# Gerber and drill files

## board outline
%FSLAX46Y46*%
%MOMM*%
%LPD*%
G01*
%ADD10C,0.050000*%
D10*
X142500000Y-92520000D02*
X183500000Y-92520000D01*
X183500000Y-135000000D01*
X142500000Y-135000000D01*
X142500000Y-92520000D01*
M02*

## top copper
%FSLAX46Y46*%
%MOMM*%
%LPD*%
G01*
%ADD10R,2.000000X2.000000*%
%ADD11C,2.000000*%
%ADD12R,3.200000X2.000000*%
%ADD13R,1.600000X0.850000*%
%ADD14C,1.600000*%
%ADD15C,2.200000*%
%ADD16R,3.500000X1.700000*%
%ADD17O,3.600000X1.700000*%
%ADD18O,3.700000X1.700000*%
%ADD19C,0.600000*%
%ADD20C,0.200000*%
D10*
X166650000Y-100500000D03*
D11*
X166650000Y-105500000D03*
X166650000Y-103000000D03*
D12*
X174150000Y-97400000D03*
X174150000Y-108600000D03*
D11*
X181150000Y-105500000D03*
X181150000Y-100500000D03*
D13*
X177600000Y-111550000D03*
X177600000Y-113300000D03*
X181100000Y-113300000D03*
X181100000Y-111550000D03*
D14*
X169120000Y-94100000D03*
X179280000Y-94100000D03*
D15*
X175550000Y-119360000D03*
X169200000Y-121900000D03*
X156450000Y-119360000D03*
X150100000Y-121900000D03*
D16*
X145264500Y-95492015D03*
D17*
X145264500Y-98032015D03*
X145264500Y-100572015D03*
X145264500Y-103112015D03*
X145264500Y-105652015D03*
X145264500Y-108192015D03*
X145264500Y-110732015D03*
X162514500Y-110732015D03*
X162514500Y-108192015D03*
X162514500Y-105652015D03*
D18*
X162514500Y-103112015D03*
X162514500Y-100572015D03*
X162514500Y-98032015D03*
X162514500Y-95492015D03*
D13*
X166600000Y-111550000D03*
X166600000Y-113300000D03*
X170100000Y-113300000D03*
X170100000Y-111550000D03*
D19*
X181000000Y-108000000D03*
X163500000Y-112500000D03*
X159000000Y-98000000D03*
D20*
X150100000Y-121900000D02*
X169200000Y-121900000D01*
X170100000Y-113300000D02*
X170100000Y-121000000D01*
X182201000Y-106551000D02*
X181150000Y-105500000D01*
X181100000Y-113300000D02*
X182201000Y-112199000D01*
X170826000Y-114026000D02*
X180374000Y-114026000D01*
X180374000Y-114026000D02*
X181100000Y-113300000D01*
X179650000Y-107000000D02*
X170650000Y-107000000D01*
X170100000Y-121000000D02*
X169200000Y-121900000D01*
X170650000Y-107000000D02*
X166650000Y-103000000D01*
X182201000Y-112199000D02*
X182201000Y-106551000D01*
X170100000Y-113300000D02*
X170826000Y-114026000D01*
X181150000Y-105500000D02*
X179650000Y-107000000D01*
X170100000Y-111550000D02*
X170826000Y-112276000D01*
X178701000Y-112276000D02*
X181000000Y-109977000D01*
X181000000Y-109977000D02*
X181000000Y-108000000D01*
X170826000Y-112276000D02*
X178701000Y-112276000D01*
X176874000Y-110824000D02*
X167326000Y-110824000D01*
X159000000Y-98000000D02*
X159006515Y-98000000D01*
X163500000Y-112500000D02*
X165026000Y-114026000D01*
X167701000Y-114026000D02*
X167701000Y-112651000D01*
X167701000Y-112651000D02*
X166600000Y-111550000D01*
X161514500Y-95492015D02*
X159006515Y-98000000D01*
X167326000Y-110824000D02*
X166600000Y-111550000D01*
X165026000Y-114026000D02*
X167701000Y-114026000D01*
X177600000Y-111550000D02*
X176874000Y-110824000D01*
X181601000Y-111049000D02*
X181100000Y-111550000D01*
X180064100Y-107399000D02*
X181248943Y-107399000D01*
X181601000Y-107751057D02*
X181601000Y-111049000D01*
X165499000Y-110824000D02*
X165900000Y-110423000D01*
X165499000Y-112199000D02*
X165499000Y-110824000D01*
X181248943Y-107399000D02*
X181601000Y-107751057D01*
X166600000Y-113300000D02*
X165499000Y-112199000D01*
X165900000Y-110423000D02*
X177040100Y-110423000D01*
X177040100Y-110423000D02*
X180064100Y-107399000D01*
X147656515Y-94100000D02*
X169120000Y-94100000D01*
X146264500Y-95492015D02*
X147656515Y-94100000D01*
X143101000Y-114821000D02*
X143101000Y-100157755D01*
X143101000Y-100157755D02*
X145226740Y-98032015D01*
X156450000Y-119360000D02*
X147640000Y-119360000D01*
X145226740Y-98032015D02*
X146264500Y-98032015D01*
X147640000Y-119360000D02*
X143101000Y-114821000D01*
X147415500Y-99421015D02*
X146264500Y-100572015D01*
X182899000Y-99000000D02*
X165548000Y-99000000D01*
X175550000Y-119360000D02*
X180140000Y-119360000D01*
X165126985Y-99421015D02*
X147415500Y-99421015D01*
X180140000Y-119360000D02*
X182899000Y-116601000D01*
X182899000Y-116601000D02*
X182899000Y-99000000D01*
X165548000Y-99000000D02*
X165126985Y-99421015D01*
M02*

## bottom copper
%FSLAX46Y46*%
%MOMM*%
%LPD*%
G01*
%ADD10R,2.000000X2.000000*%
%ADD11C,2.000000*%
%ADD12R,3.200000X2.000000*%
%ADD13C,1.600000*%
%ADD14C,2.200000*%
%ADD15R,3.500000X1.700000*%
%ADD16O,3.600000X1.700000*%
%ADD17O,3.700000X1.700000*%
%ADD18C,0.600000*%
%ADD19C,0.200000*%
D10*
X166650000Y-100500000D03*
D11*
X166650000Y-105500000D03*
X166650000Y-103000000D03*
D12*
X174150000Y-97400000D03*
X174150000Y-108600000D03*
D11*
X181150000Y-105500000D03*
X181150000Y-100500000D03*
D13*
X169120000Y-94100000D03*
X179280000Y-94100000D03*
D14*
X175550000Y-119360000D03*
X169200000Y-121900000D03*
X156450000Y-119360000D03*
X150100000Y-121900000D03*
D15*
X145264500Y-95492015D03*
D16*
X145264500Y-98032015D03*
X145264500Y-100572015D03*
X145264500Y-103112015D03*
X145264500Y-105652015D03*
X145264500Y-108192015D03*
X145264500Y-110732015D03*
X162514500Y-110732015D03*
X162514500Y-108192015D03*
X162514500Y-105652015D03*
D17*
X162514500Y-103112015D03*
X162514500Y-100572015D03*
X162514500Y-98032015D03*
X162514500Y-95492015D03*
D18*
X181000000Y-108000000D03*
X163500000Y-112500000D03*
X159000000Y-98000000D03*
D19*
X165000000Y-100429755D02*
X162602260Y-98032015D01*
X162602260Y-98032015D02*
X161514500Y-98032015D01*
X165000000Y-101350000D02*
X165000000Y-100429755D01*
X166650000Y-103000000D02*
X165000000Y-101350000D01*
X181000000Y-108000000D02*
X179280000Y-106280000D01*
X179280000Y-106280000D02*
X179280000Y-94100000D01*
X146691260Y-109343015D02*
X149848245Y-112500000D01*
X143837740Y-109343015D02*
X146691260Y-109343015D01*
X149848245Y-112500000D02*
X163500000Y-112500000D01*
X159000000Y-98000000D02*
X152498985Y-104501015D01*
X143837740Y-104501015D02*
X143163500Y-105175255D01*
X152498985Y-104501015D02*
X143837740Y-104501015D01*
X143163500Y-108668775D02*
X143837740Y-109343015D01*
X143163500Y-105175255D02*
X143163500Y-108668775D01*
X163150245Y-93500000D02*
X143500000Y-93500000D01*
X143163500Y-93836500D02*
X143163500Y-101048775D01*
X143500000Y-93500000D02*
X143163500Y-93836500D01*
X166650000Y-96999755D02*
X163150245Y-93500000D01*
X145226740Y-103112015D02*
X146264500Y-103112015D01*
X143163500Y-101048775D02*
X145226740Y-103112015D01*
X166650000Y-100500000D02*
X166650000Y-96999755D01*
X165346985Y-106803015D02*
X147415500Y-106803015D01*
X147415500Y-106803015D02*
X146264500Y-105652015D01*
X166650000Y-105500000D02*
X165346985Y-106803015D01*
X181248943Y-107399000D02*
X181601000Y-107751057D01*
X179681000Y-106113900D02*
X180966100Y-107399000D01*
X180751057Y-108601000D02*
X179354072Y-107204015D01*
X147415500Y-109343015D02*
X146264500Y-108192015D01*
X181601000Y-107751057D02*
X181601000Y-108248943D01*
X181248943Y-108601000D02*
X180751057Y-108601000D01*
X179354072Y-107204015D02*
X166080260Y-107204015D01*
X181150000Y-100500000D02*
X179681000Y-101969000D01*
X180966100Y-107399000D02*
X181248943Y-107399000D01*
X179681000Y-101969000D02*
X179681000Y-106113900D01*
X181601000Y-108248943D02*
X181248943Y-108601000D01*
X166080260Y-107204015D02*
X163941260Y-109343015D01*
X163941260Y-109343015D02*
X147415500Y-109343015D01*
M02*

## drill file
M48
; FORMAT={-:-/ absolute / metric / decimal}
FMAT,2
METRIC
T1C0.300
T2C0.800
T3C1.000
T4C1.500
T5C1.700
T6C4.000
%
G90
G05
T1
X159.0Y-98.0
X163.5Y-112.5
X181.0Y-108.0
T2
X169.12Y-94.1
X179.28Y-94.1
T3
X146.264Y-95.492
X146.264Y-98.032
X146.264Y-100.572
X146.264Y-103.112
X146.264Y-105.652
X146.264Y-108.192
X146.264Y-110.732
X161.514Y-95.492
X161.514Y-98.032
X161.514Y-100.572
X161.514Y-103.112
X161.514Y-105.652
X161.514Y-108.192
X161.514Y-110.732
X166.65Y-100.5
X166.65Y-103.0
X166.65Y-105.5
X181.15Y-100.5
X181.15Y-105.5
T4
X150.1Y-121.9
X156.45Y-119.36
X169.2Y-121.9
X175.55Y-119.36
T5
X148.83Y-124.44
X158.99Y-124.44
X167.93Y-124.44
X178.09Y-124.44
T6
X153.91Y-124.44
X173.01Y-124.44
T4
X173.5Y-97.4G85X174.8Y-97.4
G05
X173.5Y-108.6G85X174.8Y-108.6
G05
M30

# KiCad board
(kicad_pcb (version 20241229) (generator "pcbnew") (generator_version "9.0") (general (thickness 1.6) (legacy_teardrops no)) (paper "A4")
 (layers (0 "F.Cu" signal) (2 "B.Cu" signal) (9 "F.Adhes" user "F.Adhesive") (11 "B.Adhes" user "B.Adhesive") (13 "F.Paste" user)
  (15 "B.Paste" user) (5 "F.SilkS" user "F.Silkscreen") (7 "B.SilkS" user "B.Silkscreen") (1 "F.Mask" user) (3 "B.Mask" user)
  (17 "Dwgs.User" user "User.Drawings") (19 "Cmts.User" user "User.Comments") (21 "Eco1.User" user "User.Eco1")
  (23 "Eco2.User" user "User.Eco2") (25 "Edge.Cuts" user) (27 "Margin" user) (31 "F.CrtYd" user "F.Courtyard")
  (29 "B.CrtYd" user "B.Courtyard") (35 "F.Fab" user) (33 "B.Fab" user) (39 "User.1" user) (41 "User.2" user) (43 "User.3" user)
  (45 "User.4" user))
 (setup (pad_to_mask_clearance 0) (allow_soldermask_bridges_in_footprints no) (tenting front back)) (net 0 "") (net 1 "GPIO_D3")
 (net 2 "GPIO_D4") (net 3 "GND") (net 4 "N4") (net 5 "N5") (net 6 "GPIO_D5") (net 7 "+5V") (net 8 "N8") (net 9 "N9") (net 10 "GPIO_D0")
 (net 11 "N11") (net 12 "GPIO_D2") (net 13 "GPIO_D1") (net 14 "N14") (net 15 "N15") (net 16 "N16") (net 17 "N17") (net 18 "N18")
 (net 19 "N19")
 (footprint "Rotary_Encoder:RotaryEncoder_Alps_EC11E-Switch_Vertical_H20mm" (layer "F.Cu") (at 166.65 100.5)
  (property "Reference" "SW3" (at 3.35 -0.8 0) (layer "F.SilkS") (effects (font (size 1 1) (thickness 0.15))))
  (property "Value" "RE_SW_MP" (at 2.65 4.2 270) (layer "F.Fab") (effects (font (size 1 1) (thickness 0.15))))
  (pad "A" thru_hole rect (at 0 0) (size 2 2) (drill 1) (layers "*.Cu" "*.Mask") (remove_unused_layers no) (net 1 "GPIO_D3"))
  (pad "B" thru_hole circle (at 0 5) (size 2 2) (drill 1) (layers "*.Cu" "*.Mask") (remove_unused_layers no) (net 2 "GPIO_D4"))
  (pad "C" thru_hole circle (at 0 2.5) (size 2 2) (drill 1) (layers "*.Cu" "*.Mask") (remove_unused_layers no) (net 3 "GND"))
  (pad "MP" thru_hole rect (at 7.5 -3.1) (size 3.2 2) (drill oval 2.8 1.5) (layers "*.Cu" "*.Mask") (remove_unused_layers no) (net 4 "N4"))
  (pad "MP" thru_hole rect (at 7.5 8.1) (size 3.2 2) (drill oval 2.8 1.5) (layers "*.Cu" "*.Mask") (remove_unused_layers no) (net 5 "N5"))
  (pad "S1" thru_hole circle (at 14.5 5) (size 2 2) (drill 1) (layers "*.Cu" "*.Mask") (remove_unused_layers no) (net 3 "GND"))
  (pad "S2" thru_hole circle (at 14.5 0) (size 2 2) (drill 1) (layers "*.Cu" "*.Mask") (remove_unused_layers no) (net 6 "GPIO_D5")))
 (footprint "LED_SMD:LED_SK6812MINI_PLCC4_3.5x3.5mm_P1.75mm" (layer "F.Cu") (at 179.35 112.425)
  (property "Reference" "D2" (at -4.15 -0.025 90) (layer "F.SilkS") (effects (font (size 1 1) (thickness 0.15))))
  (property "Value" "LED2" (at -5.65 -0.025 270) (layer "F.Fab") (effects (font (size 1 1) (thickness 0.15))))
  (pad "1" smd rect (at -1.75 -0.875) (size 1.6 0.85) (layers "F.Cu" "F.Mask" "F.Paste") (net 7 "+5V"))
  (pad "2" smd rect (at -1.75 0.875) (size 1.6 0.85) (layers "F.Cu" "F.Mask" "F.Paste") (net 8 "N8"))
  (pad "3" smd rect (at 1.75 0.875) (size 1.6 0.85) (layers "F.Cu" "F.Mask" "F.Paste") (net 3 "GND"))
  (pad "4" smd rect (at 1.75 -0.875) (size 1.6 0.85) (layers "F.Cu" "F.Mask" "F.Paste") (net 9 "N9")))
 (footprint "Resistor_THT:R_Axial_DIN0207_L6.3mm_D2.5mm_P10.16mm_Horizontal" (layer "F.Cu") (at 169.12 94.1)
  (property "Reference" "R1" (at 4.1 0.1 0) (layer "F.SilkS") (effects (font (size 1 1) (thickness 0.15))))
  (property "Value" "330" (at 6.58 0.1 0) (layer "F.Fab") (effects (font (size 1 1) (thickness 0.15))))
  (pad "1" thru_hole circle (at 0 0) (size 1.6 1.6) (drill 0.8) (layers "*.Cu" "*.Mask") (remove_unused_layers no) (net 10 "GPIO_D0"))
  (pad "2" thru_hole circle (at 10.16 0) (size 1.6 1.6) (drill 0.8) (layers "*.Cu" "*.Mask") (remove_unused_layers no) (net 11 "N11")))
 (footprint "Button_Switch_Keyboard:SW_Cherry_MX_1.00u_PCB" (layer "F.Cu") (at 175.55 119.36)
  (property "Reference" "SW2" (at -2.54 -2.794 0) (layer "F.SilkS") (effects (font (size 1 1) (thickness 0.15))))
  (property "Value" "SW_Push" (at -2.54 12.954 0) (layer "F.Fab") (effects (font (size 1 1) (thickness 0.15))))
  (pad "" np_thru_hole circle (at -7.62 5.08) (size 1.7 1.7) (drill 1.7) (layers "*.Cu" "*.Mask"))
  (pad "" np_thru_hole circle (at -2.54 5.08) (size 4 4) (drill 4) (layers "*.Cu" "*.Mask"))
  (pad "" np_thru_hole circle (at 2.54 5.08) (size 1.7 1.7) (drill 1.7) (layers "*.Cu" "*.Mask"))
  (pad "1" thru_hole circle (at 0 0) (size 2.2 2.2) (drill 1.5) (layers "*.Cu" "*.Mask") (remove_unused_layers no) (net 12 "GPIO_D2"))
  (pad "2" thru_hole circle (at -6.35 2.54) (size 2.2 2.2) (drill 1.5) (layers "*.Cu" "*.Mask") (remove_unused_layers no) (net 3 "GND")))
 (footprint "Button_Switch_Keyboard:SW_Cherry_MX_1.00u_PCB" (layer "F.Cu") (at 156.45 119.36)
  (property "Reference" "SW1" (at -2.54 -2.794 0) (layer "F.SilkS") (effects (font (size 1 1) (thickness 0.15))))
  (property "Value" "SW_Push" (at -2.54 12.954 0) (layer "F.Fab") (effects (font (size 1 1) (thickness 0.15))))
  (pad "" np_thru_hole circle (at -7.62 5.08) (size 1.7 1.7) (drill 1.7) (layers "*.Cu" "*.Mask"))
  (pad "" np_thru_hole circle (at -2.54 5.08) (size 4 4) (drill 4) (layers "*.Cu" "*.Mask"))
  (pad "" np_thru_hole circle (at 2.54 5.08) (size 1.7 1.7) (drill 1.7) (layers "*.Cu" "*.Mask"))
  (pad "1" thru_hole circle (at 0 0) (size 2.2 2.2) (drill 1.5) (layers "*.Cu" "*.Mask") (remove_unused_layers no) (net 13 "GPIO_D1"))
  (pad "2" thru_hole circle (at -6.35 2.54) (size 2.2 2.2) (drill 1.5) (layers "*.Cu" "*.Mask") (remove_unused_layers no) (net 3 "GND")))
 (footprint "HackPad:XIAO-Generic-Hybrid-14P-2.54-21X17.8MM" (layer "F.Cu") (at 153.8895 103.112015)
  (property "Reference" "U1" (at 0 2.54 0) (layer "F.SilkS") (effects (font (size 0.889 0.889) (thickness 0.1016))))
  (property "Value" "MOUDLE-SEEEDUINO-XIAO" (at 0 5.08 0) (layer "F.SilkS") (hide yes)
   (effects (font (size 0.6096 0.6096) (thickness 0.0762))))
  (pad "1" thru_hole rect (at -7.625 -7.62) (size 3.5 1.7) (drill 1 (offset -1 0)) (layers "*.Cu" "*.Mask") (remove_unused_layers no)
   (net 10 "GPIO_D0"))
  (pad "2" thru_hole oval (at -7.625 -5.08) (size 3.6 1.7) (drill 1 (offset -1 0)) (layers "*.Cu" "*.Mask") (remove_unused_layers no)
   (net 13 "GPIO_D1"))
  (pad "3" thru_hole oval (at -7.625 -2.54) (size 3.6 1.7) (drill 1 (offset -1 0)) (layers "*.Cu" "*.Mask") (remove_unused_layers no)
   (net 12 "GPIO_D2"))
  (pad "4" thru_hole oval (at -7.625 0) (size 3.6 1.7) (drill 1 (offset -1 0)) (layers "*.Cu" "*.Mask") (remove_unused_layers no)
   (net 1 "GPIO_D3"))
  (pad "5" thru_hole oval (at -7.625 2.54) (size 3.6 1.7) (drill 1 (offset -1 0)) (layers "*.Cu" "*.Mask") (remove_unused_layers no)
   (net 2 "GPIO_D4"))
  (pad "6" thru_hole oval (at -7.625 5.08 180) (size 3.6 1.7) (drill 1 (offset 1 0)) (layers "*.Cu" "*.Mask") (remove_unused_layers no)
   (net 6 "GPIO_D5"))
  (pad "7" thru_hole oval (at -7.625 7.62) (size 3.6 1.7) (drill 1 (offset -1 0)) (layers "*.Cu" "*.Mask") (remove_unused_layers no)
   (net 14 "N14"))
  (pad "8" thru_hole oval (at 7.625 7.62) (size 3.6 1.7) (drill 1 (offset 1 0)) (layers "*.Cu" "*.Mask") (remove_unused_layers no)
   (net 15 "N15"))
  (pad "9" thru_hole oval (at 7.625 5.08) (size 3.6 1.7) (drill 1 (offset 1 0)) (layers "*.Cu" "*.Mask") (remove_unused_layers no)
   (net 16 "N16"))
  (pad "10" thru_hole oval (at 7.625 2.54) (size 3.6 1.7) (drill 1 (offset 1 0)) (layers "*.Cu" "*.Mask") (remove_unused_layers no)
   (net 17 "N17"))
  (pad "11" thru_hole oval (at 7.625 0) (size 3.7 1.7) (drill 1 (offset 1 0)) (layers "*.Cu" "*.Mask") (remove_unused_layers no)
   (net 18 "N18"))
  (pad "12" thru_hole oval (at 7.625 -2.54) (size 3.7 1.7) (drill 1 (offset 1 0)) (layers "*.Cu" "*.Mask") (remove_unused_layers no)
   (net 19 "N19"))
  (pad "13" thru_hole oval (at 7.625 -5.08) (size 3.7 1.7) (drill 1 (offset 1 0)) (layers "*.Cu" "*.Mask") (remove_unused_layers no)
   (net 3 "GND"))
  (pad "14" thru_hole oval (at 7.625 -7.62) (size 3.7 1.7) (drill 1 (offset 1 0)) (layers "*.Cu" "*.Mask") (remove_unused_layers no)
   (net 7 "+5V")))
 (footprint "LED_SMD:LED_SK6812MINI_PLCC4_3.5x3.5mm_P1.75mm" (layer "F.Cu") (at 168.35 112.425)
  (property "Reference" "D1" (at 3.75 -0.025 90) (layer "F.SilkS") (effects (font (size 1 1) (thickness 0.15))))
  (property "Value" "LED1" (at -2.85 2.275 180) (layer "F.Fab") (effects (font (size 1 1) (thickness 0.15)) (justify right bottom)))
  (pad "1" smd rect (at -1.75 -0.875) (size 1.6 0.85) (layers "F.Cu" "F.Mask" "F.Paste") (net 7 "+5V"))
  (pad "2" smd rect (at -1.75 0.875) (size 1.6 0.85) (layers "F.Cu" "F.Mask" "F.Paste") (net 9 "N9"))
  (pad "3" smd rect (at 1.75 0.875) (size 1.6 0.85) (layers "F.Cu" "F.Mask" "F.Paste") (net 3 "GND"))
  (pad "4" smd rect (at 1.75 -0.875) (size 1.6 0.85) (layers "F.Cu" "F.Mask" "F.Paste") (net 11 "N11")))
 (gr_rect (start 142.5 92.52) (end 183.5 135) (stroke (width 0.05) (type default)) (fill no) (layer "Edge.Cuts"))
 (segment (start 150.1 121.9) (end 169.2 121.9) (width 0.2) (layer "F.Cu") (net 3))
 (segment (start 170.1 113.3) (end 170.1 121) (width 0.2) (layer "F.Cu") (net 3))
 (segment (start 182.201 106.551) (end 181.15 105.5) (width 0.2) (layer "F.Cu") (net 3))
 (segment (start 181.1 113.3) (end 182.201 112.199) (width 0.2) (layer "F.Cu") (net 3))
 (segment (start 170.826 114.026) (end 180.374 114.026) (width 0.2) (layer "F.Cu") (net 3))
 (segment (start 180.374 114.026) (end 181.1 113.3) (width 0.2) (layer "F.Cu") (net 3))
 (segment (start 179.65 107) (end 170.65 107) (width 0.2) (layer "F.Cu") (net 3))
 (segment (start 170.1 121) (end 169.2 121.9) (width 0.2) (layer "F.Cu") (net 3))
 (segment (start 170.65 107) (end 166.65 103) (width 0.2) (layer "F.Cu") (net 3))
 (segment (start 182.201 112.199) (end 182.201 106.551) (width 0.2) (layer "F.Cu") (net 3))
 (segment (start 170.1 113.3) (end 170.826 114.026) (width 0.2) (layer "F.Cu") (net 3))
 (segment (start 181.15 105.5) (end 179.65 107) (width 0.2) (layer "F.Cu") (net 3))
 (segment (start 165 100.429755) (end 162.60226 98.032015) (width 0.2) (layer "B.Cu") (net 3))
 (segment (start 162.60226 98.032015) (end 161.5145 98.032015) (width 0.2) (layer "B.Cu") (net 3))
 (segment (start 165 101.35) (end 165 100.429755) (width 0.2) (layer "B.Cu") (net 3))
 (segment (start 166.65 103) (end 165 101.35) (width 0.2) (layer "B.Cu") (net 3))
 (segment (start 170.1 111.55) (end 170.826 112.276) (width 0.2) (layer "F.Cu") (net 11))
 (segment (start 178.701 112.276) (end 181 109.977) (width 0.2) (layer "F.Cu") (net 11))
 (segment (start 181 109.977) (end 181 108) (width 0.2) (layer "F.Cu") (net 11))
 (segment (start 170.826 112.276) (end 178.701 112.276) (width 0.2) (layer "F.Cu") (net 11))
 (via (at 181 108) (size 0.6) (drill 0.3) (layers "F.Cu" "B.Cu") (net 11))
 (segment (start 181 108) (end 179.28 106.28) (width 0.2) (layer "B.Cu") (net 11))
 (segment (start 179.28 106.28) (end 179.28 94.1) (width 0.2) (layer "B.Cu") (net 11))
 (segment (start 176.874 110.824) (end 167.326 110.824) (width 0.2) (layer "F.Cu") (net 7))
 (segment (start 159 98) (end 159.006515 98) (width 0.2) (layer "F.Cu") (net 7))
 (segment (start 163.5 112.5) (end 165.026 114.026) (width 0.2) (layer "F.Cu") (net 7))
 (segment (start 167.701 114.026) (end 167.701 112.651) (width 0.2) (layer "F.Cu") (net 7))
 (segment (start 167.701 112.651) (end 166.6 111.55) (width 0.2) (layer "F.Cu") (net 7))
 (segment (start 161.5145 95.492015) (end 159.006515 98) (width 0.2) (layer "F.Cu") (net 7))
 (segment (start 167.326 110.824) (end 166.6 111.55) (width 0.2) (layer "F.Cu") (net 7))
 (segment (start 165.026 114.026) (end 167.701 114.026) (width 0.2) (layer "F.Cu") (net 7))
 (segment (start 177.6 111.55) (end 176.874 110.824) (width 0.2) (layer "F.Cu") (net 7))
 (via (at 163.5 112.5) (size 0.6) (drill 0.3) (layers "F.Cu" "B.Cu") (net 7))
 (via (at 159 98) (size 0.6) (drill 0.3) (layers "F.Cu" "B.Cu") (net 7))
 (segment (start 146.69126 109.343015) (end 149.848245 112.5) (width 0.2) (layer "B.Cu") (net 7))
 (segment (start 143.83774 109.343015) (end 146.69126 109.343015) (width 0.2) (layer "B.Cu") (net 7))
 (segment (start 149.848245 112.5) (end 163.5 112.5) (width 0.2) (layer "B.Cu") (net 7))
 (segment (start 159 98) (end 152.498985 104.501015) (width 0.2) (layer "B.Cu") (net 7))
 (segment (start 143.83774 104.501015) (end 143.1635 105.175255) (width 0.2) (layer "B.Cu") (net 7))
 (segment (start 152.498985 104.501015) (end 143.83774 104.501015) (width 0.2) (layer "B.Cu") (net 7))
 (segment (start 143.1635 108.668775) (end 143.83774 109.343015) (width 0.2) (layer "B.Cu") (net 7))
 (segment (start 143.1635 105.175255) (end 143.1635 108.668775) (width 0.2) (layer "B.Cu") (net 7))
 (segment (start 181.601 111.049) (end 181.1 111.55) (width 0.2) (layer "F.Cu") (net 9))
 (segment (start 180.0641 107.399) (end 181.248943 107.399) (width 0.2) (layer "F.Cu") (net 9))
 (segment (start 181.601 107.751057) (end 181.601 111.049) (width 0.2) (layer "F.Cu") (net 9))
 (segment (start 165.499 110.824) (end 165.9 110.423) (width 0.2) (layer "F.Cu") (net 9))
 (segment (start 165.499 112.199) (end 165.499 110.824) (width 0.2) (layer "F.Cu") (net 9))
 (segment (start 181.248943 107.399) (end 181.601 107.751057) (width 0.2) (layer "F.Cu") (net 9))
 (segment (start 166.6 113.3) (end 165.499 112.199) (width 0.2) (layer "F.Cu") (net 9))
 (segment (start 165.9 110.423) (end 177.0401 110.423) (width 0.2) (layer "F.Cu") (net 9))
 (segment (start 177.0401 110.423) (end 180.0641 107.399) (width 0.2) (layer "F.Cu") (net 9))
 (segment (start 147.656515 94.1) (end 169.12 94.1) (width 0.2) (layer "F.Cu") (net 10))
 (segment (start 146.2645 95.492015) (end 147.656515 94.1) (width 0.2) (layer "F.Cu") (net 10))
 (segment (start 143.101 114.821) (end 143.101 100.157755) (width 0.2) (layer "F.Cu") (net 13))
 (segment (start 143.101 100.157755) (end 145.22674 98.032015) (width 0.2) (layer "F.Cu") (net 13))
 (segment (start 156.45 119.36) (end 147.64 119.36) (width 0.2) (layer "F.Cu") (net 13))
 (segment (start 145.22674 98.032015) (end 146.2645 98.032015) (width 0.2) (layer "F.Cu") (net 13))
 (segment (start 147.64 119.36) (end 143.101 114.821) (width 0.2) (layer "F.Cu") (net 13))
 (segment (start 147.4155 99.421015) (end 146.2645 100.572015) (width 0.2) (layer "F.Cu") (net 12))
 (segment (start 182.899 99) (end 165.548 99) (width 0.2) (layer "F.Cu") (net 12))
 (segment (start 175.55 119.36) (end 180.14 119.36) (width 0.2) (layer "F.Cu") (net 12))
 (segment (start 165.126985 99.421015) (end 147.4155 99.421015) (width 0.2) (layer "F.Cu") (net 12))
 (segment (start 180.14 119.36) (end 182.899 116.601) (width 0.2) (layer "F.Cu") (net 12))
 (segment (start 182.899 116.601) (end 182.899 99) (width 0.2) (layer "F.Cu") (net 12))
 (segment (start 165.548 99) (end 165.126985 99.421015) (width 0.2) (layer "F.Cu") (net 12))
 (segment (start 163.150245 93.5) (end 143.5 93.5) (width 0.2) (layer "B.Cu") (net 1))
 (segment (start 143.1635 93.8365) (end 143.1635 101.048775) (width 0.2) (layer "B.Cu") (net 1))
 (segment (start 143.5 93.5) (end 143.1635 93.8365) (width 0.2) (layer "B.Cu") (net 1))
 (segment (start 166.65 96.999755) (end 163.150245 93.5) (width 0.2) (layer "B.Cu") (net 1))
 (segment (start 145.22674 103.112015) (end 146.2645 103.112015) (width 0.2) (layer "B.Cu") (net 1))
 (segment (start 143.1635 101.048775) (end 145.22674 103.112015) (width 0.2) (layer "B.Cu") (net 1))
 (segment (start 166.65 100.5) (end 166.65 96.999755) (width 0.2) (layer "B.Cu") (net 1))
 (segment (start 165.346985 106.803015) (end 147.4155 106.803015) (width 0.2) (layer "B.Cu") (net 2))
 (segment (start 147.4155 106.803015) (end 146.2645 105.652015) (width 0.2) (layer "B.Cu") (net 2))
 (segment (start 166.65 105.5) (end 165.346985 106.803015) (width 0.2) (layer "B.Cu") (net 2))
 (segment (start 181.248943 107.399) (end 181.601 107.751057) (width 0.2) (layer "B.Cu") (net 6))
 (segment (start 179.681 106.1139) (end 180.9661 107.399) (width 0.2) (layer "B.Cu") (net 6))
 (segment (start 180.751057 108.601) (end 179.354072 107.204015) (width 0.2) (layer "B.Cu") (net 6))
 (segment (start 147.4155 109.343015) (end 146.2645 108.192015) (width 0.2) (layer "B.Cu") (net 6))
 (segment (start 181.601 107.751057) (end 181.601 108.248943) (width 0.2) (layer "B.Cu") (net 6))
 (segment (start 181.248943 108.601) (end 180.751057 108.601) (width 0.2) (layer "B.Cu") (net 6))
 (segment (start 179.354072 107.204015) (end 166.08026 107.204015) (width 0.2) (layer "B.Cu") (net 6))
 (segment (start 181.15 100.5) (end 179.681 101.969) (width 0.2) (layer "B.Cu") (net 6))
 (segment (start 180.9661 107.399) (end 181.248943 107.399) (width 0.2) (layer "B.Cu") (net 6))
 (segment (start 179.681 101.969) (end 179.681 106.1139) (width 0.2) (layer "B.Cu") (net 6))
 (segment (start 181.601 108.248943) (end 181.248943 108.601) (width 0.2) (layer "B.Cu") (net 6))
 (segment (start 166.08026 107.204015) (end 163.94126 109.343015) (width 0.2) (layer "B.Cu") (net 6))
 (segment (start 163.94126 109.343015) (end 147.4155 109.343015) (width 0.2) (layer "B.Cu") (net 6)))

